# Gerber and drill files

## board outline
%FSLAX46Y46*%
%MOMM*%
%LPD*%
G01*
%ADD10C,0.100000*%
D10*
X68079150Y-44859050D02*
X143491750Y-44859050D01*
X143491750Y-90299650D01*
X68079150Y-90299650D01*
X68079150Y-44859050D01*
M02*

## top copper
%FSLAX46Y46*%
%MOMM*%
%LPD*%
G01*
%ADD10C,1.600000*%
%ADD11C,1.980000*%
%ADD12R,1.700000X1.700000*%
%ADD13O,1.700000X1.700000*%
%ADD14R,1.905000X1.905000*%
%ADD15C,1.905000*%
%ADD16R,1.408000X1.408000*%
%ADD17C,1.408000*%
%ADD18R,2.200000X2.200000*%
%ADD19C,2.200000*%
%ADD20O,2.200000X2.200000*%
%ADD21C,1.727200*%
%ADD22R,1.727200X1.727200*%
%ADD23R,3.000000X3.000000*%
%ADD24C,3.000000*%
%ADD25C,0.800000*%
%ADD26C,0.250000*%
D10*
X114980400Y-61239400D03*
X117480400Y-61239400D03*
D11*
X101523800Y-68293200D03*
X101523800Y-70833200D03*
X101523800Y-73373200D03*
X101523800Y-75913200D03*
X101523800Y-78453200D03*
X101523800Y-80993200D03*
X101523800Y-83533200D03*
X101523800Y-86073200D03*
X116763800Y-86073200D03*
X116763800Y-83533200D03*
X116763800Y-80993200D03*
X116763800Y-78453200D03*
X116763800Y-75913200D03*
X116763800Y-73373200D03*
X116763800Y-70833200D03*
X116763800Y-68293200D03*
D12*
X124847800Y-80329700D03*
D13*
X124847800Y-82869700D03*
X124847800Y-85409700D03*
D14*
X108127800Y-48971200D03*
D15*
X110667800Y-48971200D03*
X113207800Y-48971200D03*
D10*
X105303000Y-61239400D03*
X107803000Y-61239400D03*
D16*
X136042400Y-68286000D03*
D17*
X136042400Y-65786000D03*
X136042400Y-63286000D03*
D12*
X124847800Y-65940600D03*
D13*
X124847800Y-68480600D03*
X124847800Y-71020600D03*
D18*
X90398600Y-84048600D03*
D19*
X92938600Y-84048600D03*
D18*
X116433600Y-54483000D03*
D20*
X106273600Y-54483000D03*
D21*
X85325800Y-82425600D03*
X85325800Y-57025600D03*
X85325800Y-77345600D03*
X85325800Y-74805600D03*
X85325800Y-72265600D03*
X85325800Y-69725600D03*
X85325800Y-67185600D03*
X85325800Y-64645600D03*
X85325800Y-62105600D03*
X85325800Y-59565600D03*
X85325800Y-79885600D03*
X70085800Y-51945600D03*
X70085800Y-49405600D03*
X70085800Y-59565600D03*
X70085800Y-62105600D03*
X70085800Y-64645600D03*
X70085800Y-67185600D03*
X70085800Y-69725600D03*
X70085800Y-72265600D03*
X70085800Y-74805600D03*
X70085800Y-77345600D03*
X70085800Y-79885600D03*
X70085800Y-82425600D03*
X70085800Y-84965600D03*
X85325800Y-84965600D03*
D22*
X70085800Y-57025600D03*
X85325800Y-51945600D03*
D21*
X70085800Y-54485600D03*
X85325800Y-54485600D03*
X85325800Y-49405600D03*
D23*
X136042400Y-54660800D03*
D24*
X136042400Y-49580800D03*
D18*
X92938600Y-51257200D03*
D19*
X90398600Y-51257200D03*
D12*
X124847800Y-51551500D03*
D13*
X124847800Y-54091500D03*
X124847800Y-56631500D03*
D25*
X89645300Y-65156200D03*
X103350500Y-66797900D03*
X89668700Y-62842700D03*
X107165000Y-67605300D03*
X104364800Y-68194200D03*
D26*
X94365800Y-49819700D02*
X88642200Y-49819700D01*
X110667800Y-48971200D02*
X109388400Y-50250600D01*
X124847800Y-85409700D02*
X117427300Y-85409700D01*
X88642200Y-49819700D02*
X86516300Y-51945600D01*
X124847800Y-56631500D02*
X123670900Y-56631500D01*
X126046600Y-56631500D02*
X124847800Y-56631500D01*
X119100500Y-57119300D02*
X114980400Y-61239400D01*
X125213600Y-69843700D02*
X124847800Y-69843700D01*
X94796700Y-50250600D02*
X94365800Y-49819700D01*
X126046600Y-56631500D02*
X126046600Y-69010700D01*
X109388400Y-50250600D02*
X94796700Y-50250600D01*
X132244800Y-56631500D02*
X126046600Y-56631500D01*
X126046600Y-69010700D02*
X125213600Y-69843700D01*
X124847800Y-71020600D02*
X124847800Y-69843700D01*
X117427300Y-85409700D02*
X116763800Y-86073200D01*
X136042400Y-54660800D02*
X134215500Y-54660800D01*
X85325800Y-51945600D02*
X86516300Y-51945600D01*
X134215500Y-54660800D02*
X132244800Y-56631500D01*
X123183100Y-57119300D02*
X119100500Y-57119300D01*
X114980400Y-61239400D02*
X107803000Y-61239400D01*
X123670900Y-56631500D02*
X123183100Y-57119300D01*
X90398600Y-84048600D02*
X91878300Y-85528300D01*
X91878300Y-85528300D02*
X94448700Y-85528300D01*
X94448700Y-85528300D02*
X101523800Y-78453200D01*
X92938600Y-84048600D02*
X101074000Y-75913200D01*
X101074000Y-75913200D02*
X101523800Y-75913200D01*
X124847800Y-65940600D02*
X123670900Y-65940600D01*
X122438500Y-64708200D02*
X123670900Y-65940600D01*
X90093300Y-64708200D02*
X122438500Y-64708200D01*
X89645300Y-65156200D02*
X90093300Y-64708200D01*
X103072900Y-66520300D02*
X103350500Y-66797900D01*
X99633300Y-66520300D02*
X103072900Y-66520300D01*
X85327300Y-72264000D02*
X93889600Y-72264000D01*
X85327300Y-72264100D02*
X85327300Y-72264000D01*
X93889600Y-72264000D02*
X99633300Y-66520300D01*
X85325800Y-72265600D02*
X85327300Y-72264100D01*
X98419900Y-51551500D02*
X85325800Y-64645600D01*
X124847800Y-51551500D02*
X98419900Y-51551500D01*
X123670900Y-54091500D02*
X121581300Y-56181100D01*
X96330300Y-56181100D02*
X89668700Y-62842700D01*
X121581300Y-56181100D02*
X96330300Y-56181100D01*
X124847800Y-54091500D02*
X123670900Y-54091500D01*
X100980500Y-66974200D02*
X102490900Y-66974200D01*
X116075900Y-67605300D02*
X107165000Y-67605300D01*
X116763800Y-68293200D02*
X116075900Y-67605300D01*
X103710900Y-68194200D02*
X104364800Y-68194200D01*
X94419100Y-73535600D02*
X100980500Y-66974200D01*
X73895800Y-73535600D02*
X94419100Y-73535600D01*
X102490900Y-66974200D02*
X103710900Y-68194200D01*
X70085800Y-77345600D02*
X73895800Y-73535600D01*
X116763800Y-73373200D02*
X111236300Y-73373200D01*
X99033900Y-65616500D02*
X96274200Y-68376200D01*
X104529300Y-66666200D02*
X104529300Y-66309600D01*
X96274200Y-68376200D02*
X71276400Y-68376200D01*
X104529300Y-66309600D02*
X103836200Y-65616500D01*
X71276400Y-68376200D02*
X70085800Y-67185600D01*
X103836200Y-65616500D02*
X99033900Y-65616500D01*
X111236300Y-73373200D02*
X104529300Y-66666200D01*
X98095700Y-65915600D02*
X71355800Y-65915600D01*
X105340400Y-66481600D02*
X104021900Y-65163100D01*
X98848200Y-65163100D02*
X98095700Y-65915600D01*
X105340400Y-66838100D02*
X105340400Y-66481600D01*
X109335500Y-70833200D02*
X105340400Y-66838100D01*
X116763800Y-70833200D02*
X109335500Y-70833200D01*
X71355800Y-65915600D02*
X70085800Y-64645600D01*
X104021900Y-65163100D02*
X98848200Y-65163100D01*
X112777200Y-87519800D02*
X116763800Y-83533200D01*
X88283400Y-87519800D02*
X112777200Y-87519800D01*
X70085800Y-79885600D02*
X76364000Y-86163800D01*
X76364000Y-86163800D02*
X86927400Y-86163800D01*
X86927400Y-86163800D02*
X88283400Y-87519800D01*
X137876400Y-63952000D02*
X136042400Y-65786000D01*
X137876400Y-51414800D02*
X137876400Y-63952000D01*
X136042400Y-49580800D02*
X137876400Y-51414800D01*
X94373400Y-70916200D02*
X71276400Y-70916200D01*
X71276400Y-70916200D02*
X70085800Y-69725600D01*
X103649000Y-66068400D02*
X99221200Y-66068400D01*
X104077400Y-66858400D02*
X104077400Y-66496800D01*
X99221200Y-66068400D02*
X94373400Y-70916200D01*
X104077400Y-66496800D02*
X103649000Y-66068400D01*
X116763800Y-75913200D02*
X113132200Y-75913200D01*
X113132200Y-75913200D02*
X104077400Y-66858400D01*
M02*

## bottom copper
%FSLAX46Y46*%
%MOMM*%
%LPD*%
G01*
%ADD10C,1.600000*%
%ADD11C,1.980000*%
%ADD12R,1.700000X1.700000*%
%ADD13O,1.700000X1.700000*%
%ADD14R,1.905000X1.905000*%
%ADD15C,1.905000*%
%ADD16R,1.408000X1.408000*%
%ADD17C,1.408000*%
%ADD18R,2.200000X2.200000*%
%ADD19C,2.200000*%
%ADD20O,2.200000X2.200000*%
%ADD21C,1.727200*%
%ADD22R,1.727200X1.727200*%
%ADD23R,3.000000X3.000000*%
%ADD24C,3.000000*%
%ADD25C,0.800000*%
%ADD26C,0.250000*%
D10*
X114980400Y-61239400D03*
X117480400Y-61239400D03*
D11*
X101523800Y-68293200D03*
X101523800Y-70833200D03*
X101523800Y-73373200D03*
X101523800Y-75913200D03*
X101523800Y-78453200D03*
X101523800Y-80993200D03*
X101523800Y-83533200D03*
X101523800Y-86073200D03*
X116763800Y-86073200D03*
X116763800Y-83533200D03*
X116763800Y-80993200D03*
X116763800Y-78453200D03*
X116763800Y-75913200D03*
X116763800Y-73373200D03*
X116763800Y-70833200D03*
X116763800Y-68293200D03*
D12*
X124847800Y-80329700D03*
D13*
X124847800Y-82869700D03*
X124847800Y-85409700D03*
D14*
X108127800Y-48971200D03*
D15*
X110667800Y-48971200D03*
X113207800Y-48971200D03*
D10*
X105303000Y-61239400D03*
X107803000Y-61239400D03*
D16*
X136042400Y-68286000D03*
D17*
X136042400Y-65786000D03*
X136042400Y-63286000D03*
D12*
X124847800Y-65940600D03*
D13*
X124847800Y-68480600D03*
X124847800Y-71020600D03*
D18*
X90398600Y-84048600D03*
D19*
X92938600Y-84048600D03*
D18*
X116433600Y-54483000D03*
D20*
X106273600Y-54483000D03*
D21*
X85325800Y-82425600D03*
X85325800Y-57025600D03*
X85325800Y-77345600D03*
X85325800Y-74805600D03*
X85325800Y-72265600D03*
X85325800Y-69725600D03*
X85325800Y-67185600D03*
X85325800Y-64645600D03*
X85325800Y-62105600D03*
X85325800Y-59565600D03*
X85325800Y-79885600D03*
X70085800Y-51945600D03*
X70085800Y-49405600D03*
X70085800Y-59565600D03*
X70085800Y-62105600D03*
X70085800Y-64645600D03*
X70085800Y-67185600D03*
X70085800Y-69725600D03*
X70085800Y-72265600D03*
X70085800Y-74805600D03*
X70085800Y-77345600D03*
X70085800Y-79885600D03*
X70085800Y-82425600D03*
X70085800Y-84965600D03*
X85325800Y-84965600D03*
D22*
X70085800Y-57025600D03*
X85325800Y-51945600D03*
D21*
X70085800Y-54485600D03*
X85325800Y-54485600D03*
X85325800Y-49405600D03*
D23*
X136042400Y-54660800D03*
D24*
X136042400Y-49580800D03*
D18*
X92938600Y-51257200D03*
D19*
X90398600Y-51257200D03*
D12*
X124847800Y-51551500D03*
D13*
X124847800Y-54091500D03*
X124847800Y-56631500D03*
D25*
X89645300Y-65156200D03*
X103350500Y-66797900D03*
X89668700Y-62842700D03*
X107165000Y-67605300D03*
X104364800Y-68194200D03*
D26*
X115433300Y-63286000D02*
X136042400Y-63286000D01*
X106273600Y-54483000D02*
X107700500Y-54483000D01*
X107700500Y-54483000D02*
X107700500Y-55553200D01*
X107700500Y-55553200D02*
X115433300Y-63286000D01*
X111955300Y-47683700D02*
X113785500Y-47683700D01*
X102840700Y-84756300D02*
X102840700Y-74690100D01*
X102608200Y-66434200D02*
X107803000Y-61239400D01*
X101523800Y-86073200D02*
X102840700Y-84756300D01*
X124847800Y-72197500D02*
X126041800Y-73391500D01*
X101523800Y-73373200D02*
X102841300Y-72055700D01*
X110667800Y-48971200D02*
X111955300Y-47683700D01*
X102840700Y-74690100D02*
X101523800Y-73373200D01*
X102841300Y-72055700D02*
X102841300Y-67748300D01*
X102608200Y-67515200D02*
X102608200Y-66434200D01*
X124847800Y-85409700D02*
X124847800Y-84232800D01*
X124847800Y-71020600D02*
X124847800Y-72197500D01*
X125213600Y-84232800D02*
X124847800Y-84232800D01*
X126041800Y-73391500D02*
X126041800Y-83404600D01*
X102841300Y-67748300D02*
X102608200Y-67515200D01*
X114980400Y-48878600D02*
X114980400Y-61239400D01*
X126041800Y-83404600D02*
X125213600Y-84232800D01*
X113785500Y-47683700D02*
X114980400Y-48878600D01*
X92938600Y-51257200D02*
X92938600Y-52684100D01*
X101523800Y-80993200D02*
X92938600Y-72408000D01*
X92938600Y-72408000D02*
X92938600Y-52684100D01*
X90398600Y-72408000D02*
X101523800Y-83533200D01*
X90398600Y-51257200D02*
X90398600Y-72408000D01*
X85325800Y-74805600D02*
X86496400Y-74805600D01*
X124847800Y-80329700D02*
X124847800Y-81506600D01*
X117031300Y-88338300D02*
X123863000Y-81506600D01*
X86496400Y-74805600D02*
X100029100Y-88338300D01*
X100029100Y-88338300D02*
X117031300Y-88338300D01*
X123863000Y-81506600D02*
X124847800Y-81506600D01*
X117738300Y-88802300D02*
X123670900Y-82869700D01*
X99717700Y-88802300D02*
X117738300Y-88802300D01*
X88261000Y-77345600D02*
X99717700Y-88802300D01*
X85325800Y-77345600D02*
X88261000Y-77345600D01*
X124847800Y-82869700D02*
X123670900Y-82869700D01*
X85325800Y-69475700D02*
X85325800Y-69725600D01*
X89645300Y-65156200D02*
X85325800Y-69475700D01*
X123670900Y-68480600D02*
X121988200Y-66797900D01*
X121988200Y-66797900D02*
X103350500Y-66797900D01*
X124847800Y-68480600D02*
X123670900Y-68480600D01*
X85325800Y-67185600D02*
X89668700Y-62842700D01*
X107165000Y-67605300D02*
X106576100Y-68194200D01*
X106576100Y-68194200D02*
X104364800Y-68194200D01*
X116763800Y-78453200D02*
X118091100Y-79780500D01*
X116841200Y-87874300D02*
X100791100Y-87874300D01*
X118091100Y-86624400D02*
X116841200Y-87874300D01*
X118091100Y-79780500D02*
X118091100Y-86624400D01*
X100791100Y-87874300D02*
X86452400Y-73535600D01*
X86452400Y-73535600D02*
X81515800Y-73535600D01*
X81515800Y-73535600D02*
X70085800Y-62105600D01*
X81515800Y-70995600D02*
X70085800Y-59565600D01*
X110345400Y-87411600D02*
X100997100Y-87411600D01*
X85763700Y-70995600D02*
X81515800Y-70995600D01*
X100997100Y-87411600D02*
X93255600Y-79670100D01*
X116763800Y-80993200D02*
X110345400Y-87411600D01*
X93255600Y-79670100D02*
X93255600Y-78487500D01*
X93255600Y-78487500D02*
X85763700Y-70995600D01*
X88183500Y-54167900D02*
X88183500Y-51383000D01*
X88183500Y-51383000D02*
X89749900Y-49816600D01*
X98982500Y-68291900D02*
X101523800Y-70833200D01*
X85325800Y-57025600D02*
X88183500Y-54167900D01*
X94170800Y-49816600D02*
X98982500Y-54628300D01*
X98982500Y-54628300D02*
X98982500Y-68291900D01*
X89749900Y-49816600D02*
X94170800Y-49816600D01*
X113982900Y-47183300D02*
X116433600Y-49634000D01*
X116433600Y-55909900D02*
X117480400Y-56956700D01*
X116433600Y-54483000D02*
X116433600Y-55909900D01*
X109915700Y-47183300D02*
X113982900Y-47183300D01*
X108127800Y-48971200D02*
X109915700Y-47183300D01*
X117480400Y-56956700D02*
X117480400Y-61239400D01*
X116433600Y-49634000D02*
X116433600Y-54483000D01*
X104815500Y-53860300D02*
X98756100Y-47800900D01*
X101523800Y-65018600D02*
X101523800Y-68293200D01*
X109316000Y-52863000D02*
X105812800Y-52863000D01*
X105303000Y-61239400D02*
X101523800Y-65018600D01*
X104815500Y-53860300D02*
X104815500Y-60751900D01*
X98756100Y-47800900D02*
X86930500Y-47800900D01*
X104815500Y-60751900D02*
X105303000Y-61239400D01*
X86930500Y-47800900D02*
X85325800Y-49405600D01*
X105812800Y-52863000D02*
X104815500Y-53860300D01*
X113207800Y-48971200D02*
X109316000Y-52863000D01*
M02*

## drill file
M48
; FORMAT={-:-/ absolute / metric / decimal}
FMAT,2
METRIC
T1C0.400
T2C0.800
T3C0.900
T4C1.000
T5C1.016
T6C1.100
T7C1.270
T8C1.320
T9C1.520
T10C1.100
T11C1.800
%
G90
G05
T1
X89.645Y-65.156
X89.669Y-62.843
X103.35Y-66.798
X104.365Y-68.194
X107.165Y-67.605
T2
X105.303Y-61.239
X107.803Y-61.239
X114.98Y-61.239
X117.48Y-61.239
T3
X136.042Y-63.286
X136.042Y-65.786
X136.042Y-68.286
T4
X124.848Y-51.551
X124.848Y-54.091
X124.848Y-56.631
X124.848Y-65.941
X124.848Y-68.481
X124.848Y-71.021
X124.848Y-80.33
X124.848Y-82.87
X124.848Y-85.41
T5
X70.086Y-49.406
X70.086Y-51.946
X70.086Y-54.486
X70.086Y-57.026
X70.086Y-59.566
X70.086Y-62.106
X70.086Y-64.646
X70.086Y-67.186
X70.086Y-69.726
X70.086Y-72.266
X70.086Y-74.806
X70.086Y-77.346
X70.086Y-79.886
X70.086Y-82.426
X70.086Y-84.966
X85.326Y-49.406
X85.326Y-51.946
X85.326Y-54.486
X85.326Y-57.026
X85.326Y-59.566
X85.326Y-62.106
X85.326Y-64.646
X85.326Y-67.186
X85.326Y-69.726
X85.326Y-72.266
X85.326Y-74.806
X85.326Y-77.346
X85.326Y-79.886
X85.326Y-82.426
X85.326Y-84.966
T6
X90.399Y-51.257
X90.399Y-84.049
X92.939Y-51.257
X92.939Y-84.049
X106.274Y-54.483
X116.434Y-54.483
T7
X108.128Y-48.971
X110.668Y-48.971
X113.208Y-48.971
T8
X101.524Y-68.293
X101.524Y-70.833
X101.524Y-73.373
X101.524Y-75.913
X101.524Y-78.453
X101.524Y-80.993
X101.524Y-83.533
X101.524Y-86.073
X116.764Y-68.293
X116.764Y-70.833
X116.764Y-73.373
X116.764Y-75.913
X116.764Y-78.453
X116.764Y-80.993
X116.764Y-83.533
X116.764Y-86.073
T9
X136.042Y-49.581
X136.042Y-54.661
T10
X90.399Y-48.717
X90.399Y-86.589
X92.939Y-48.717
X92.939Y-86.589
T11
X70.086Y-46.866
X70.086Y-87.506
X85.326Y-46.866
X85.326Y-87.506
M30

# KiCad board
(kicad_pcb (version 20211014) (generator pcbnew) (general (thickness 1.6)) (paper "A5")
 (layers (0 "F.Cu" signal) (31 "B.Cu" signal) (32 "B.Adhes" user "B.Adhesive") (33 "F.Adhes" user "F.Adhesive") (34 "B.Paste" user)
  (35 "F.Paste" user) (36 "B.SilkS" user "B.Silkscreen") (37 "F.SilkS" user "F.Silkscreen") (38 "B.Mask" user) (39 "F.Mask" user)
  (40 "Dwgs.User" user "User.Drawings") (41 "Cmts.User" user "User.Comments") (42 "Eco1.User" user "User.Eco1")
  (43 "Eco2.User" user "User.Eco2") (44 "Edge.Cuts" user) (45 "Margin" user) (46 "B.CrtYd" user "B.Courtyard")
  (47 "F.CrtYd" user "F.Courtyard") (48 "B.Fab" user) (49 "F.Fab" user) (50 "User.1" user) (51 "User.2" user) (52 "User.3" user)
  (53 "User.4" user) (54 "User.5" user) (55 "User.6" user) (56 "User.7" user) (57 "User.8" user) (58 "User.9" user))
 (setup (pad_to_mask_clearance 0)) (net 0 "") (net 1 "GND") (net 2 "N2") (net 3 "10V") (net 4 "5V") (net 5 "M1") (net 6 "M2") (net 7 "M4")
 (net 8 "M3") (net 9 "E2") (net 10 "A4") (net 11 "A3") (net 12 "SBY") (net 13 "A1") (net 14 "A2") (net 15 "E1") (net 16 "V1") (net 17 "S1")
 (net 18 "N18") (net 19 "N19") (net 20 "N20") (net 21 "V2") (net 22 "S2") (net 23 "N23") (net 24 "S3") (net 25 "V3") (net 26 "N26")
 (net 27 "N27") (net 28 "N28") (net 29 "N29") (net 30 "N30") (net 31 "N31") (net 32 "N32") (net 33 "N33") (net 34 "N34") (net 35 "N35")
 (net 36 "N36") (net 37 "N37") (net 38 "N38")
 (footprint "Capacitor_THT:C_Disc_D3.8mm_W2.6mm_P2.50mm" (layer "F.Cu") (at 114.9804 61.2394)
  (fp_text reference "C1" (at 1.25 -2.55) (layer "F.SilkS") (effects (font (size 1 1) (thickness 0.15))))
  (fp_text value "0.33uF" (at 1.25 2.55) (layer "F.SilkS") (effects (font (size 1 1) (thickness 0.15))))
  (pad "1" thru_hole circle (at 0 0) (size 1.6 1.6) (drill 0.8) (layers *.Cu *.Mask) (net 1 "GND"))
  (pad "2" thru_hole circle (at 2.5 0) (size 1.6 1.6) (drill 0.8) (layers *.Cu *.Mask) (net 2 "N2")))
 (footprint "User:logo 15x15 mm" (layer "F.Cu") (at 136.972523 80.725423)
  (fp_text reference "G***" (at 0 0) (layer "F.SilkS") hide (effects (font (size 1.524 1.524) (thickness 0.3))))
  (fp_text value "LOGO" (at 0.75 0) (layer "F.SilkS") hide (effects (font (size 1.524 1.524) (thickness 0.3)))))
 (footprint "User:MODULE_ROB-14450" (layer "F.Cu") (at 109.1438 77.1832)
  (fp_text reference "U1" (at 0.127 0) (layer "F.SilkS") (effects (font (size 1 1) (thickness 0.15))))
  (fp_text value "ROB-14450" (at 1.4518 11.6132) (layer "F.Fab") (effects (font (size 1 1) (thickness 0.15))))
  (pad "1" thru_hole circle locked (at -7.62 -8.89) (size 1.98 1.98) (drill 1.32) (layers *.Cu *.Mask) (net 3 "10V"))
  (pad "2" thru_hole circle locked (at -7.62 -6.35) (size 1.98 1.98) (drill 1.32) (layers *.Cu *.Mask) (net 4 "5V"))
  (pad "3" thru_hole circle locked (at -7.62 -3.81) (size 1.98 1.98) (drill 1.32) (layers *.Cu *.Mask) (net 1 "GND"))
  (pad "4" thru_hole circle locked (at -7.62 -1.27) (size 1.98 1.98) (drill 1.32) (layers *.Cu *.Mask) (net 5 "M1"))
  (pad "5" thru_hole circle locked (at -7.62 1.27) (size 1.98 1.98) (drill 1.32) (layers *.Cu *.Mask) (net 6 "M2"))
  (pad "6" thru_hole circle locked (at -7.62 3.81) (size 1.98 1.98) (drill 1.32) (layers *.Cu *.Mask) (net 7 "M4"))
  (pad "7" thru_hole circle locked (at -7.62 6.35) (size 1.98 1.98) (drill 1.32) (layers *.Cu *.Mask) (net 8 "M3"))
  (pad "8" thru_hole circle locked (at -7.62 8.89) (size 1.98 1.98) (drill 1.32) (layers *.Cu *.Mask) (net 1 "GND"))
  (pad "9" thru_hole circle locked (at 7.62 8.89) (size 1.98 1.98) (drill 1.32) (layers *.Cu *.Mask) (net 1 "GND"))
  (pad "10" thru_hole circle locked (at 7.62 6.35) (size 1.98 1.98) (drill 1.32) (layers *.Cu *.Mask) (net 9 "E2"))
  (pad "11" thru_hole circle locked (at 7.62 3.81) (size 1.98 1.98) (drill 1.32) (layers *.Cu *.Mask) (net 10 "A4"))
  (pad "12" thru_hole circle locked (at 7.62 1.27) (size 1.98 1.98) (drill 1.32) (layers *.Cu *.Mask) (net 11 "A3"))
  (pad "13" thru_hole circle locked (at 7.62 -1.27) (size 1.98 1.98) (drill 1.32) (layers *.Cu *.Mask) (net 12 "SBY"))
  (pad "14" thru_hole circle locked (at 7.62 -3.81) (size 1.98 1.98) (drill 1.32) (layers *.Cu *.Mask) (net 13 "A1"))
  (pad "15" thru_hole circle locked (at 7.62 -6.35) (size 1.98 1.98) (drill 1.32) (layers *.Cu *.Mask) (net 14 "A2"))
  (pad "16" thru_hole circle locked (at 7.62 -8.89) (size 1.98 1.98) (drill 1.32) (layers *.Cu *.Mask) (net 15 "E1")))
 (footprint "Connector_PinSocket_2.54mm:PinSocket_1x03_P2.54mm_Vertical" (layer "F.Cu") (at 124.8478 80.3297)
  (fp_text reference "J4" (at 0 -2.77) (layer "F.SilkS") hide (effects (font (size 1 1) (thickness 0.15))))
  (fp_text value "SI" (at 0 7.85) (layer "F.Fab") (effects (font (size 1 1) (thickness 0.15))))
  (pad "1" thru_hole rect (at 0 0) (size 1.7 1.7) (drill 1) (layers *.Cu *.Mask) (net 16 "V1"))
  (pad "2" thru_hole oval (at 0 2.54) (size 1.7 1.7) (drill 1) (layers *.Cu *.Mask) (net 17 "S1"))
  (pad "3" thru_hole oval (at 0 5.08) (size 1.7 1.7) (drill 1) (layers *.Cu *.Mask) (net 1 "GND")))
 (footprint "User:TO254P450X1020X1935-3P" (layer "F.Cu") (at 113.2078 47.879)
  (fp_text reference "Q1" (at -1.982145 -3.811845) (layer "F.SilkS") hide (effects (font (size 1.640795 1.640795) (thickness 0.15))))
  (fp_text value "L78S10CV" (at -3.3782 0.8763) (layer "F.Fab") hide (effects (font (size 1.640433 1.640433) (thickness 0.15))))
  (pad "1" thru_hole rect locked (at -5.08 1.0922) (size 1.905 1.905) (drill 1.27) (layers *.Cu *.Mask) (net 2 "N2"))
  (pad "2" thru_hole circle locked (at -2.54 1.0922) (size 1.905 1.905) (drill 1.27) (layers *.Cu *.Mask) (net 1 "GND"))
  (pad "3" thru_hole circle locked (at 0 1.0922) (size 1.905 1.905) (drill 1.27) (layers *.Cu *.Mask) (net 3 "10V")))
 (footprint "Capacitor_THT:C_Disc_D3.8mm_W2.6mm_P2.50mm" (layer "F.Cu") (at 105.303 61.2394)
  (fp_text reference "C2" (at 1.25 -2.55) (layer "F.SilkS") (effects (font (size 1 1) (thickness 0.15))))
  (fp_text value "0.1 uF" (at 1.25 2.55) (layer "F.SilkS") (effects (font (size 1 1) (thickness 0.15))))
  (pad "1" thru_hole circle (at 0 0) (size 1.6 1.6) (drill 0.8) (layers *.Cu *.Mask) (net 3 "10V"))
  (pad "2" thru_hole circle (at 2.5 0) (size 1.6 1.6) (drill 0.8) (layers *.Cu *.Mask) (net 1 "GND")))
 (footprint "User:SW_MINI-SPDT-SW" (layer "F.Cu") (at 136.0424 65.786 90)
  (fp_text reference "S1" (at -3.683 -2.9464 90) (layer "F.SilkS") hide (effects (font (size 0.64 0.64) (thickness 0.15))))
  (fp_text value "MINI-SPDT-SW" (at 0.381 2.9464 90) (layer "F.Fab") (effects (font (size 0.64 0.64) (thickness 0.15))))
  (pad "1" thru_hole rect locked (at -2.5 0 90) (size 1.408 1.408) (drill 0.9) (layers *.Cu *.Mask) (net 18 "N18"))
  (pad "2" thru_hole circle locked (at 0 0 90) (size 1.408 1.408) (drill 0.9) (layers *.Cu *.Mask) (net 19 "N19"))
  (pad "3" thru_hole circle locked (at 2.5 0 90) (size 1.408 1.408) (drill 0.9) (layers *.Cu *.Mask) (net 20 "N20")))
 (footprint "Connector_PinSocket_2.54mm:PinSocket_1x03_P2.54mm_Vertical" (layer "F.Cu") (at 124.8478 65.9406)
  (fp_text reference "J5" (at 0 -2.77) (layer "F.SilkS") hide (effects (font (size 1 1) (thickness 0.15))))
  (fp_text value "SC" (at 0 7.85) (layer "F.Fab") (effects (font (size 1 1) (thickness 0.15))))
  (pad "1" thru_hole rect (at 0 0) (size 1.7 1.7) (drill 1) (layers *.Cu *.Mask) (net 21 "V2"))
  (pad "2" thru_hole oval (at 0 2.54) (size 1.7 1.7) (drill 1) (layers *.Cu *.Mask) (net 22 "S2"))
  (pad "3" thru_hole oval (at 0 5.08) (size 1.7 1.7) (drill 1) (layers *.Cu *.Mask) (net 1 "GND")))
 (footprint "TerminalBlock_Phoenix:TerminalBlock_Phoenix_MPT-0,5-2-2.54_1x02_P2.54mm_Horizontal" (layer "F.Cu") (at 90.3986 84.0486)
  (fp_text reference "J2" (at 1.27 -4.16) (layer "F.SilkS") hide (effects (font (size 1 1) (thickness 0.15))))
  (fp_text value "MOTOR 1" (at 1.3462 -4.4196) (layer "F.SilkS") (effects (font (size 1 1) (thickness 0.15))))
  (pad "" np_thru_hole circle (at 2.54 2.54) (size 1.1 1.1) (drill 1.1) (layers *.Cu *.Mask))
  (pad "" np_thru_hole circle (at 0 2.54) (size 1.1 1.1) (drill 1.1) (layers *.Cu *.Mask))
  (pad "1" thru_hole rect (at 0 0) (size 2.2 2.2) (drill 1.1) (layers *.Cu *.Mask) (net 6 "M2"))
  (pad "2" thru_hole circle (at 2.54 0) (size 2.2 2.2) (drill 1.1) (layers *.Cu *.Mask) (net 5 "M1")))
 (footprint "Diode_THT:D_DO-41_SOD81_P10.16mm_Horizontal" (layer "F.Cu") (at 116.4336 54.483 180)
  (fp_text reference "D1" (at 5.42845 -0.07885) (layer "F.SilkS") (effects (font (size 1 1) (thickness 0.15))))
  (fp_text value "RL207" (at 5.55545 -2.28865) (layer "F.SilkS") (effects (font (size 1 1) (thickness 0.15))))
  (pad "1" thru_hole rect (at 0 0 180) (size 2.2 2.2) (drill 1.1) (layers *.Cu *.Mask) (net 2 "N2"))
  (pad "2" thru_hole oval (at 10.16 0 180) (size 2.2 2.2) (drill 1.1) (layers *.Cu *.Mask) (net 20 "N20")))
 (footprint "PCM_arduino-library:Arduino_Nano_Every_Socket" (layer "F.Cu") (at 77.7058 88.7756)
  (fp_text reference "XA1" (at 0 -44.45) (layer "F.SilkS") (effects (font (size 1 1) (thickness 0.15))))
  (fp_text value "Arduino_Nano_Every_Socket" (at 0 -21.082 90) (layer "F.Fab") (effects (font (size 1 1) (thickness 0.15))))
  (pad "" np_thru_hole circle (at -7.62 -41.91) (size 1.8 1.8) (drill 1.8) (layers F&B.Cu *.Mask))
  (pad "" np_thru_hole circle (at 7.62 -1.27) (size 1.8 1.8) (drill 1.8) (layers F&B.Cu *.Mask))
  (pad "" np_thru_hole circle (at -7.62 -1.27) (size 1.8 1.8) (drill 1.8) (layers F&B.Cu *.Mask))
  (pad "" np_thru_hole circle (at 7.62 -41.91) (size 1.8 1.8) (drill 1.8) (layers F&B.Cu *.Mask))
  (pad "3V3" thru_hole circle (at 7.62 -6.35) (size 1.7272 1.7272) (drill 1.016) (layers *.Cu *.Mask) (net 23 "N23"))
  (pad "5V" thru_hole circle (at 7.62 -31.75) (size 1.7272 1.7272) (drill 1.016) (layers *.Cu *.Mask) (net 4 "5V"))
  (pad "A0" thru_hole circle (at 7.62 -11.43) (size 1.7272 1.7272) (drill 1.016) (layers *.Cu *.Mask) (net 17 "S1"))
  (pad "A1" thru_hole circle (at 7.62 -13.97) (size 1.7272 1.7272) (drill 1.016) (layers *.Cu *.Mask) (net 16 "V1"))
  (pad "A2" thru_hole circle (at 7.62 -16.51) (size 1.7272 1.7272) (drill 1.016) (layers *.Cu *.Mask) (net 22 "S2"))
  (pad "A3" thru_hole circle (at 7.62 -19.05) (size 1.7272 1.7272) (drill 1.016) (layers *.Cu *.Mask) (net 21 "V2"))
  (pad "A4" thru_hole circle (at 7.62 -21.59) (size 1.7272 1.7272) (drill 1.016) (layers *.Cu *.Mask) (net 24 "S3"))
  (pad "A5" thru_hole circle (at 7.62 -24.13) (size 1.7272 1.7272) (drill 1.016) (layers *.Cu *.Mask) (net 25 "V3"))
  (pad "A6" thru_hole circle (at 7.62 -26.67) (size 1.7272 1.7272) (drill 1.016) (layers *.Cu *.Mask) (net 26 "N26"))
  (pad "A7" thru_hole circle (at 7.62 -29.21) (size 1.7272 1.7272) (drill 1.016) (layers *.Cu *.Mask) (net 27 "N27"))
  (pad "AREF" thru_hole circle (at 7.62 -8.89) (size 1.7272 1.7272) (drill 1.016) (layers *.Cu *.Mask) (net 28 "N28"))
  (pad "D0" thru_hole circle (at -7.62 -36.83) (size 1.7272 1.7272) (drill 1.016) (layers *.Cu *.Mask) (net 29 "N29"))
  (pad "D1" thru_hole circle (at -7.62 -39.37) (size 1.7272 1.7272) (drill 1.016) (layers *.Cu *.Mask) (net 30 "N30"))
  (pad "D2" thru_hole circle (at -7.62 -29.21) (size 1.7272 1.7272) (drill 1.016) (layers *.Cu *.Mask) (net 10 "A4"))
  (pad "D3" thru_hole circle (at -7.62 -26.67) (size 1.7272 1.7272) (drill 1.016) (layers *.Cu *.Mask) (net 11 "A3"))
  (pad "D4" thru_hole circle (at -7.62 -24.13) (size 1.7272 1.7272) (drill 1.016) (layers *.Cu *.Mask) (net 14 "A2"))
  (pad "D5" thru_hole circle (at -7.62 -21.59) (size 1.7272 1.7272) (drill 1.016) (layers *.Cu *.Mask) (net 13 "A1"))
  (pad "D6" thru_hole circle (at -7.62 -19.05) (size 1.7272 1.7272) (drill 1.016) (layers *.Cu *.Mask) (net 12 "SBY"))
  (pad "D7" thru_hole circle (at -7.62 -16.51) (size 1.7272 1.7272) (drill 1.016) (layers *.Cu *.Mask) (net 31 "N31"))
  (pad "D8" thru_hole circle (at -7.62 -13.97) (size 1.7272 1.7272) (drill 1.016) (layers *.Cu *.Mask) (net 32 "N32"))
  (pad "D9" thru_hole circle (at -7.62 -11.43) (size 1.7272 1.7272) (drill 1.016) (layers *.Cu *.Mask) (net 15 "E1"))
  (pad "D10" thru_hole circle (at -7.62 -8.89) (size 1.7272 1.7272) (drill 1.016) (layers *.Cu *.Mask) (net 9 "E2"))
  (pad "D11" thru_hole circle (at -7.62 -6.35) (size 1.7272 1.7272) (drill 1.016) (layers *.Cu *.Mask) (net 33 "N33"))
  (pad "D12" thru_hole circle (at -7.62 -3.81) (size 1.7272 1.7272) (drill 1.016) (layers *.Cu *.Mask) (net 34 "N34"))
  (pad "D13" thru_hole circle (at 7.62 -3.81) (size 1.7272 1.7272) (drill 1.016) (layers *.Cu *.Mask) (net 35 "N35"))
  (pad "GND1" thru_hole rect (at -7.62 -31.75) (size 1.7272 1.7272) (drill 1.016) (layers *.Cu *.Mask) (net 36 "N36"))
  (pad "GND2" thru_hole rect (at 7.62 -36.83) (size 1.7272 1.7272) (drill 1.016) (layers *.Cu *.Mask) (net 1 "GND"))
  (pad "RST1" thru_hole circle (at -7.62 -34.29) (size 1.7272 1.7272) (drill 1.016) (layers *.Cu *.Mask) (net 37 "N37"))
  (pad "RST2" thru_hole circle (at 7.62 -34.29) (size 1.7272 1.7272) (drill 1.016) (layers *.Cu *.Mask) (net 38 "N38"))
  (pad "VIN" thru_hole circle (at 7.62 -39.37) (size 1.7272 1.7272) (drill 1.016) (layers *.Cu *.Mask) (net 3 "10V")))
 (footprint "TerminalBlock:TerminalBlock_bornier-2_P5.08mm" (layer "F.Cu") (at 136.0424 54.6608 90)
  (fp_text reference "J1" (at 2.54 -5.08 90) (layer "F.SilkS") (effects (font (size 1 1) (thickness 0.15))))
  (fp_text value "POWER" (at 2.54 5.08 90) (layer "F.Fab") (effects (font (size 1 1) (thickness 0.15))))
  (pad "1" thru_hole rect (at 0 0 90) (size 3 3) (drill 1.52) (layers *.Cu *.Mask) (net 1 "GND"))
  (pad "2" thru_hole circle (at 5.08 0 90) (size 3 3) (drill 1.52) (layers *.Cu *.Mask) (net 19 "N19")))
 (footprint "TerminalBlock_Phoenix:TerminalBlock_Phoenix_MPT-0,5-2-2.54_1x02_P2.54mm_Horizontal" (layer "F.Cu") (at 92.9386 51.2572 180)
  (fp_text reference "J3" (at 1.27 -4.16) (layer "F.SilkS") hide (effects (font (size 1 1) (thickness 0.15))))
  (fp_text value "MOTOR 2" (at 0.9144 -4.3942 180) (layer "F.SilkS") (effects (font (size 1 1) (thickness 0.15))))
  (pad "" np_thru_hole circle (at 0 2.54 180) (size 1.1 1.1) (drill 1.1) (layers *.Cu *.Mask))
  (pad "" np_thru_hole circle (at 2.54 2.54 180) (size 1.1 1.1) (drill 1.1) (layers *.Cu *.Mask))
  (pad "1" thru_hole rect (at 0 0 180) (size 2.2 2.2) (drill 1.1) (layers *.Cu *.Mask) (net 7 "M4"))
  (pad "2" thru_hole circle (at 2.54 0 180) (size 2.2 2.2) (drill 1.1) (layers *.Cu *.Mask) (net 8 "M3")))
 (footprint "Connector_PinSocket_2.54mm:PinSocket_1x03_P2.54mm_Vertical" (layer "F.Cu") (at 124.8478 51.5515)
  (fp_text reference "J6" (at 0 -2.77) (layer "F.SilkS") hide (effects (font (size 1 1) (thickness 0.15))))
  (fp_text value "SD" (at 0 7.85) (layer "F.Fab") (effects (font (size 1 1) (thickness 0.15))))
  (pad "1" thru_hole rect (at 0 0) (size 1.7 1.7) (drill 1) (layers *.Cu *.Mask) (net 25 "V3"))
  (pad "2" thru_hole oval (at 0 2.54) (size 1.7 1.7) (drill 1) (layers *.Cu *.Mask) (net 24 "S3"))
  (pad "3" thru_hole oval (at 0 5.08) (size 1.7 1.7) (drill 1) (layers *.Cu *.Mask) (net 1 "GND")))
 (gr_rect (start 68.07915 44.85905) (end 143.49175 90.29965) (layer "Edge.Cuts") (width 0.1) (fill none))
 (segment (start 115.4333 63.286) (end 136.0424 63.286) (width 0.25) (layer "B.Cu") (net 20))
 (segment (start 106.2736 54.483) (end 107.7005 54.483) (width 0.25) (layer "B.Cu") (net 20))
 (segment (start 107.7005 54.483) (end 107.7005 55.5532) (width 0.25) (layer "B.Cu") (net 20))
 (segment (start 107.7005 55.5532) (end 115.4333 63.286) (width 0.25) (layer "B.Cu") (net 20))
 (segment (start 94.3658 49.8197) (end 88.6422 49.8197) (width 0.25) (layer "F.Cu") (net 1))
 (segment (start 110.6678 48.9712) (end 109.3884 50.2506) (width 0.25) (layer "F.Cu") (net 1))
 (segment (start 124.8478 85.4097) (end 117.4273 85.4097) (width 0.25) (layer "F.Cu") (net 1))
 (segment (start 88.6422 49.8197) (end 86.5163 51.9456) (width 0.25) (layer "F.Cu") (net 1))
 (segment (start 124.8478 56.6315) (end 123.6709 56.6315) (width 0.25) (layer "F.Cu") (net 1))
 (segment (start 126.0466 56.6315) (end 124.8478 56.6315) (width 0.25) (layer "F.Cu") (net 1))
 (segment (start 119.1005 57.1193) (end 114.9804 61.2394) (width 0.25) (layer "F.Cu") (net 1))
 (segment (start 125.2136 69.8437) (end 124.8478 69.8437) (width 0.25) (layer "F.Cu") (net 1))
 (segment (start 94.7967 50.2506) (end 94.3658 49.8197) (width 0.25) (layer "F.Cu") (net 1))
 (segment (start 126.0466 56.6315) (end 126.0466 69.0107) (width 0.25) (layer "F.Cu") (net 1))
 (segment (start 109.3884 50.2506) (end 94.7967 50.2506) (width 0.25) (layer "F.Cu") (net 1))
 (segment (start 132.2448 56.6315) (end 126.0466 56.6315) (width 0.25) (layer "F.Cu") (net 1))
 (segment (start 126.0466 69.0107) (end 125.2136 69.8437) (width 0.25) (layer "F.Cu") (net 1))
 (segment (start 124.8478 71.0206) (end 124.8478 69.8437) (width 0.25) (layer "F.Cu") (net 1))
 (segment (start 117.4273 85.4097) (end 116.7638 86.0732) (width 0.25) (layer "F.Cu") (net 1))
 (segment (start 136.0424 54.6608) (end 134.2155 54.6608) (width 0.25) (layer "F.Cu") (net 1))
 (segment (start 85.3258 51.9456) (end 86.5163 51.9456) (width 0.25) (layer "F.Cu") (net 1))
 (segment (start 134.2155 54.6608) (end 132.2448 56.6315) (width 0.25) (layer "F.Cu") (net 1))
 (segment (start 123.1831 57.1193) (end 119.1005 57.1193) (width 0.25) (layer "F.Cu") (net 1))
 (segment (start 114.9804 61.2394) (end 107.803 61.2394) (width 0.25) (layer "F.Cu") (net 1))
 (segment (start 123.6709 56.6315) (end 123.1831 57.1193) (width 0.25) (layer "F.Cu") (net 1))
 (segment (start 111.9553 47.6837) (end 113.7855 47.6837) (width 0.25) (layer "B.Cu") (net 1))
 (segment (start 102.8407 84.7563) (end 102.8407 74.6901) (width 0.25) (layer "B.Cu") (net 1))
 (segment (start 102.6082 66.4342) (end 107.803 61.2394) (width 0.25) (layer "B.Cu") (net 1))
 (segment (start 101.5238 86.0732) (end 102.8407 84.7563) (width 0.25) (layer "B.Cu") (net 1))
 (segment (start 124.8478 72.1975) (end 126.0418 73.3915) (width 0.25) (layer "B.Cu") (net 1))
 (segment (start 101.5238 73.3732) (end 102.8413 72.0557) (width 0.25) (layer "B.Cu") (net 1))
 (segment (start 110.6678 48.9712) (end 111.9553 47.6837) (width 0.25) (layer "B.Cu") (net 1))
 (segment (start 102.8407 74.6901) (end 101.5238 73.3732) (width 0.25) (layer "B.Cu") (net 1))
 (segment (start 102.8413 72.0557) (end 102.8413 67.7483) (width 0.25) (layer "B.Cu") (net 1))
 (segment (start 102.6082 67.5152) (end 102.6082 66.4342) (width 0.25) (layer "B.Cu") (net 1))
 (segment (start 124.8478 85.4097) (end 124.8478 84.2328) (width 0.25) (layer "B.Cu") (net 1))
 (segment (start 124.8478 71.0206) (end 124.8478 72.1975) (width 0.25) (layer "B.Cu") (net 1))
 (segment (start 125.2136 84.2328) (end 124.8478 84.2328) (width 0.25) (layer "B.Cu") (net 1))
 (segment (start 126.0418 73.3915) (end 126.0418 83.4046) (width 0.25) (layer "B.Cu") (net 1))
 (segment (start 102.8413 67.7483) (end 102.6082 67.5152) (width 0.25) (layer "B.Cu") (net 1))
 (segment (start 114.9804 48.8786) (end 114.9804 61.2394) (width 0.25) (layer "B.Cu") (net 1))
 (segment (start 126.0418 83.4046) (end 125.2136 84.2328) (width 0.25) (layer "B.Cu") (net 1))
 (segment (start 113.7855 47.6837) (end 114.9804 48.8786) (width 0.25) (layer "B.Cu") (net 1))
 (segment (start 90.3986 84.0486) (end 91.8783 85.5283) (width 0.25) (layer "F.Cu") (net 6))
 (segment (start 91.8783 85.5283) (end 94.4487 85.5283) (width 0.25) (layer "F.Cu") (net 6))
 (segment (start 94.4487 85.5283) (end 101.5238 78.4532) (width 0.25) (layer "F.Cu") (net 6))
 (segment (start 92.9386 84.0486) (end 101.074 75.9132) (width 0.25) (layer "F.Cu") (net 5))
 (segment (start 101.074 75.9132) (end 101.5238 75.9132) (width 0.25) (layer "F.Cu") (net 5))
 (segment (start 92.9386 51.2572) (end 92.9386 52.6841) (width 0.25) (layer "B.Cu") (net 7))
 (segment (start 101.5238 80.9932) (end 92.9386 72.408) (width 0.25) (layer "B.Cu") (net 7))
 (segment (start 92.9386 72.408) (end 92.9386 52.6841) (width 0.25) (layer "B.Cu") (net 7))
 (segment (start 90.3986 72.408) (end 101.5238 83.5332) (width 0.25) (layer "B.Cu") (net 8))
 (segment (start 90.3986 51.2572) (end 90.3986 72.408) (width 0.25) (layer "B.Cu") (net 8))
 (segment (start 85.3258 74.8056) (end 86.4964 74.8056) (width 0.25) (layer "B.Cu") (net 16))
 (segment (start 124.8478 80.3297) (end 124.8478 81.5066) (width 0.25) (layer "B.Cu") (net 16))
 (segment (start 117.0313 88.3383) (end 123.863 81.5066) (width 0.25) (layer "B.Cu") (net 16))
 (segment (start 86.4964 74.8056) (end 100.0291 88.3383) (width 0.25) (layer "B.Cu") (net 16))
 (segment (start 100.0291 88.3383) (end 117.0313 88.3383) (width 0.25) (layer "B.Cu") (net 16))
 (segment (start 123.863 81.5066) (end 124.8478 81.5066) (width 0.25) (layer "B.Cu") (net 16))
 (segment (start 117.7383 88.8023) (end 123.6709 82.8697) (width 0.25) (layer "B.Cu") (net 17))
 (segment (start 99.7177 88.8023) (end 117.7383 88.8023) (width 0.25) (layer "B.Cu") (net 17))
 (segment (start 88.261 77.3456) (end 99.7177 88.8023) (width 0.25) (layer "B.Cu") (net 17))
 (segment (start 85.3258 77.3456) (end 88.261 77.3456) (width 0.25) (layer "B.Cu") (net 17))
 (segment (start 124.8478 82.8697) (end 123.6709 82.8697) (width 0.25) (layer "B.Cu") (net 17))
 (segment (start 124.8478 65.9406) (end 123.6709 65.9406) (width 0.25) (layer "F.Cu") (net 21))
 (segment (start 122.4385 64.7082) (end 123.6709 65.9406) (width 0.25) (layer "F.Cu") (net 21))
 (segment (start 90.0933 64.7082) (end 122.4385 64.7082) (width 0.25) (layer "F.Cu") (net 21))
 (segment (start 89.6453 65.1562) (end 90.0933 64.7082) (width 0.25) (layer "F.Cu") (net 21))
 (via (at 89.6453 65.1562) (size 0.8) (drill 0.4) (layers "F.Cu" "B.Cu") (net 21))
 (segment (start 85.3258 69.4757) (end 85.3258 69.7256) (width 0.25) (layer "B.Cu") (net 21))
 (segment (start 89.6453 65.1562) (end 85.3258 69.4757) (width 0.25) (layer "B.Cu") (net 21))
 (segment (start 103.0729 66.5203) (end 103.3505 66.7979) (width 0.25) (layer "F.Cu") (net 22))
 (segment (start 99.6333 66.5203) (end 103.0729 66.5203) (width 0.25) (layer "F.Cu") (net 22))
 (segment (start 85.3273 72.264) (end 93.8896 72.264) (width 0.25) (layer "F.Cu") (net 22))
 (segment (start 85.3273 72.2641) (end 85.3273 72.264) (width 0.25) (layer "F.Cu") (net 22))
 (segment (start 93.8896 72.264) (end 99.6333 66.5203) (width 0.25) (layer "F.Cu") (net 22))
 (segment (start 85.3258 72.2656) (end 85.3273 72.2641) (width 0.25) (layer "F.Cu") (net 22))
 (via (at 103.3505 66.7979) (size 0.8) (drill 0.4) (layers "F.Cu" "B.Cu") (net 22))
 (segment (start 123.6709 68.4806) (end 121.9882 66.7979) (width 0.25) (layer "B.Cu") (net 22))
 (segment (start 121.9882 66.7979) (end 103.3505 66.7979) (width 0.25) (layer "B.Cu") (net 22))
 (segment (start 124.8478 68.4806) (end 123.6709 68.4806) (width 0.25) (layer "B.Cu") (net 22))
 (segment (start 98.4199 51.5515) (end 85.3258 64.6456) (width 0.25) (layer "F.Cu") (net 25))
 (segment (start 124.8478 51.5515) (end 98.4199 51.5515) (width 0.25) (layer "F.Cu") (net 25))
 (segment (start 123.6709 54.0915) (end 121.5813 56.1811) (width 0.25) (layer "F.Cu") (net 24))
 (segment (start 96.3303 56.1811) (end 89.6687 62.8427) (width 0.25) (layer "F.Cu") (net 24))
 (segment (start 121.5813 56.1811) (end 96.3303 56.1811) (width 0.25) (layer "F.Cu") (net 24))
 (segment (start 124.8478 54.0915) (end 123.6709 54.0915) (width 0.25) (layer "F.Cu") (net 24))
 (via (at 89.6687 62.8427) (size 0.8) (drill 0.4) (layers "F.Cu" "B.Cu") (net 24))
 (segment (start 85.3258 67.1856) (end 89.6687 62.8427) (width 0.25) (layer "B.Cu") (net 24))
 (segment (start 100.9805 66.9742) (end 102.4909 66.9742) (width 0.25) (layer "F.Cu") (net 15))
 (segment (start 116.0759 67.6053) (end 107.165 67.6053) (width 0.25) (layer "F.Cu") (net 15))
 (segment (start 116.7638 68.2932) (end 116.0759 67.6053) (width 0.25) (layer "F.Cu") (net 15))
 (segment (start 103.7109 68.1942) (end 104.3648 68.1942) (width 0.25) (layer "F.Cu") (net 15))
 (segment (start 94.4191 73.5356) (end 100.9805 66.9742) (width 0.25) (layer "F.Cu") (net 15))
 (segment (start 73.8958 73.5356) (end 94.4191 73.5356) (width 0.25) (layer "F.Cu") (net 15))
 (segment (start 102.4909 66.9742) (end 103.7109 68.1942) (width 0.25) (layer "F.Cu") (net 15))
 (segment (start 70.0858 77.3456) (end 73.8958 73.5356) (width 0.25) (layer "F.Cu") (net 15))
 (via (at 107.165 67.6053) (size 0.8) (drill 0.4) (layers "F.Cu" "B.Cu") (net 15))
 (via (at 104.3648 68.1942) (size 0.8) (drill 0.4) (layers "F.Cu" "B.Cu") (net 15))
 (segment (start 107.165 67.6053) (end 106.5761 68.1942) (width 0.25) (layer "B.Cu") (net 15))
 (segment (start 106.5761 68.1942) (end 104.3648 68.1942) (width 0.25) (layer "B.Cu") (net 15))
 (segment (start 116.7638 73.3732) (end 111.2363 73.3732) (width 0.25) (layer "F.Cu") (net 13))
 (segment (start 99.0339 65.6165) (end 96.2742 68.3762) (width 0.25) (layer "F.Cu") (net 13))
 (segment (start 104.5293 66.6662) (end 104.5293 66.3096) (width 0.25) (layer "F.Cu") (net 13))
 (segment (start 96.2742 68.3762) (end 71.2764 68.3762) (width 0.25) (layer "F.Cu") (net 13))
 (segment (start 104.5293 66.3096) (end 103.8362 65.6165) (width 0.25) (layer "F.Cu") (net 13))
 (segment (start 71.2764 68.3762) (end 70.0858 67.1856) (width 0.25) (layer "F.Cu") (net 13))
 (segment (start 103.8362 65.6165) (end 99.0339 65.6165) (width 0.25) (layer "F.Cu") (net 13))
 (segment (start 111.2363 73.3732) (end 104.5293 66.6662) (width 0.25) (layer "F.Cu") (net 13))
 (segment (start 98.0957 65.9156) (end 71.3558 65.9156) (width 0.25) (layer "F.Cu") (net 14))
 (segment (start 105.3404 66.4816) (end 104.0219 65.1631) (width 0.25) (layer "F.Cu") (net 14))
 (segment (start 98.8482 65.1631) (end 98.0957 65.9156) (width 0.25) (layer "F.Cu") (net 14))
 (segment (start 105.3404 66.8381) (end 105.3404 66.4816) (width 0.25) (layer "F.Cu") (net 14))
 (segment (start 109.3355 70.8332) (end 105.3404 66.8381) (width 0.25) (layer "F.Cu") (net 14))
 (segment (start 116.7638 70.8332) (end 109.3355 70.8332) (width 0.25) (layer "F.Cu") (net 14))
 (segment (start 71.3558 65.9156) (end 70.0858 64.6456) (width 0.25) (layer "F.Cu") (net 14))
 (segment (start 104.0219 65.1631) (end 98.8482 65.1631) (width 0.25) (layer "F.Cu") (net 14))
 (segment (start 112.7772 87.5198) (end 116.7638 83.5332) (width 0.25) (layer "F.Cu") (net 9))
 (segment (start 88.2834 87.5198) (end 112.7772 87.5198) (width 0.25) (layer "F.Cu") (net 9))
 (segment (start 70.0858 79.8856) (end 76.364 86.1638) (width 0.25) (layer "F.Cu") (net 9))
 (segment (start 76.364 86.1638) (end 86.9274 86.1638) (width 0.25) (layer "F.Cu") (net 9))
 (segment (start 86.9274 86.1638) (end 88.2834 87.5198) (width 0.25) (layer "F.Cu") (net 9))
 (segment (start 116.7638 78.4532) (end 118.0911 79.7805) (width 0.25) (layer "B.Cu") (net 11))
 (segment (start 116.8412 87.8743) (end 100.7911 87.8743) (width 0.25) (layer "B.Cu") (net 11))
 (segment (start 118.0911 86.6244) (end 116.8412 87.8743) (width 0.25) (layer "B.Cu") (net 11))
 (segment (start 118.0911 79.7805) (end 118.0911 86.6244) (width 0.25) (layer "B.Cu") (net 11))
 (segment (start 100.7911 87.8743) (end 86.4524 73.5356) (width 0.25) (layer "B.Cu") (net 11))
 (segment (start 86.4524 73.5356) (end 81.5158 73.5356) (width 0.25) (layer "B.Cu") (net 11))
 (segment (start 81.5158 73.5356) (end 70.0858 62.1056) (width 0.25) (layer "B.Cu") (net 11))
 (segment (start 81.5158 70.9956) (end 70.0858 59.5656) (width 0.25) (layer "B.Cu") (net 10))
 (segment (start 110.3454 87.4116) (end 100.9971 87.4116) (width 0.25) (layer "B.Cu") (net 10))
 (segment (start 85.7637 70.9956) (end 81.5158 70.9956) (width 0.25) (layer "B.Cu") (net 10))
 (segment (start 100.9971 87.4116) (end 93.2556 79.6701) (width 0.25) (layer "B.Cu") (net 10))
 (segment (start 116.7638 80.9932) (end 110.3454 87.4116) (width 0.25) (layer "B.Cu") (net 10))
 (segment (start 93.2556 79.6701) (end 93.2556 78.4875) (width 0.25) (layer "B.Cu") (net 10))
 (segment (start 93.2556 78.4875) (end 85.7637 70.9956) (width 0.25) (layer "B.Cu") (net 10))
 (segment (start 88.1835 54.1679) (end 88.1835 51.383) (width 0.25) (layer "B.Cu") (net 4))
 (segment (start 88.1835 51.383) (end 89.7499 49.8166) (width 0.25) (layer "B.Cu") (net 4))
 (segment (start 98.9825 68.2919) (end 101.5238 70.8332) (width 0.25) (layer "B.Cu") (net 4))
 (segment (start 85.3258 57.0256) (end 88.1835 54.1679) (width 0.25) (layer "B.Cu") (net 4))
 (segment (start 94.1708 49.8166) (end 98.9825 54.6283) (width 0.25) (layer "B.Cu") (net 4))
 (segment (start 98.9825 54.6283) (end 98.9825 68.2919) (width 0.25) (layer "B.Cu") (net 4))
 (segment (start 89.7499 49.8166) (end 94.1708 49.8166) (width 0.25) (layer "B.Cu") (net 4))
 (segment (start 113.9829 47.1833) (end 116.4336 49.634) (width 0.25) (layer "B.Cu") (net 2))
 (segment (start 116.4336 55.9099) (end 117.4804 56.9567) (width 0.25) (layer "B.Cu") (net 2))
 (segment (start 116.4336 54.483) (end 116.4336 55.9099) (width 0.25) (layer "B.Cu") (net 2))
 (segment (start 109.9157 47.1833) (end 113.9829 47.1833) (width 0.25) (layer "B.Cu") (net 2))
 (segment (start 108.1278 48.9712) (end 109.9157 47.1833) (width 0.25) (layer "B.Cu") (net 2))
 (segment (start 117.4804 56.9567) (end 117.4804 61.2394) (width 0.25) (layer "B.Cu") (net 2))
 (segment (start 116.4336 49.634) (end 116.4336 54.483) (width 0.25) (layer "B.Cu") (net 2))
 (segment (start 137.8764 63.952) (end 136.0424 65.786) (width 0.25) (layer "F.Cu") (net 19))
 (segment (start 137.8764 51.4148) (end 137.8764 63.952) (width 0.25) (layer "F.Cu") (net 19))
 (segment (start 136.0424 49.5808) (end 137.8764 51.4148) (width 0.25) (layer "F.Cu") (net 19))
 (segment (start 104.8155 53.8603) (end 98.7561 47.8009) (width 0.25) (layer "B.Cu") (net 3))
 (segment (start 101.5238 65.0186) (end 101.5238 68.2932) (width 0.25) (layer "B.Cu") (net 3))
 (segment (start 109.316 52.863) (end 105.8128 52.863) (width 0.25) (layer "B.Cu") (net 3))
 (segment (start 105.303 61.2394) (end 101.5238 65.0186) (width 0.25) (layer "B.Cu") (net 3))
 (segment (start 104.8155 53.8603) (end 104.8155 60.7519) (width 0.25) (layer "B.Cu") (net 3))
 (segment (start 98.7561 47.8009) (end 86.9305 47.8009) (width 0.25) (layer "B.Cu") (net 3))
 (segment (start 104.8155 60.7519) (end 105.303 61.2394) (width 0.25) (layer "B.Cu") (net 3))
 (segment (start 86.9305 47.8009) (end 85.3258 49.4056) (width 0.25) (layer "B.Cu") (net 3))
 (segment (start 105.8128 52.863) (end 104.8155 53.8603) (width 0.25) (layer "B.Cu") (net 3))
 (segment (start 113.2078 48.9712) (end 109.316 52.863) (width 0.25) (layer "B.Cu") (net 3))
 (segment (start 94.3734 70.9162) (end 71.2764 70.9162) (width 0.25) (layer "F.Cu") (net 12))
 (segment (start 71.2764 70.9162) (end 70.0858 69.7256) (width 0.25) (layer "F.Cu") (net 12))
 (segment (start 103.649 66.0684) (end 99.2212 66.0684) (width 0.25) (layer "F.Cu") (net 12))
 (segment (start 104.0774 66.8584) (end 104.0774 66.4968) (width 0.25) (layer "F.Cu") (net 12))
 (segment (start 99.2212 66.0684) (end 94.3734 70.9162) (width 0.25) (layer "F.Cu") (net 12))
 (segment (start 104.0774 66.4968) (end 103.649 66.0684) (width 0.25) (layer "F.Cu") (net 12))
 (segment (start 116.7638 75.9132) (end 113.1322 75.9132) (width 0.25) (layer "F.Cu") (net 12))
 (segment (start 113.1322 75.9132) (end 104.0774 66.8584) (width 0.25) (layer "F.Cu") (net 12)))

